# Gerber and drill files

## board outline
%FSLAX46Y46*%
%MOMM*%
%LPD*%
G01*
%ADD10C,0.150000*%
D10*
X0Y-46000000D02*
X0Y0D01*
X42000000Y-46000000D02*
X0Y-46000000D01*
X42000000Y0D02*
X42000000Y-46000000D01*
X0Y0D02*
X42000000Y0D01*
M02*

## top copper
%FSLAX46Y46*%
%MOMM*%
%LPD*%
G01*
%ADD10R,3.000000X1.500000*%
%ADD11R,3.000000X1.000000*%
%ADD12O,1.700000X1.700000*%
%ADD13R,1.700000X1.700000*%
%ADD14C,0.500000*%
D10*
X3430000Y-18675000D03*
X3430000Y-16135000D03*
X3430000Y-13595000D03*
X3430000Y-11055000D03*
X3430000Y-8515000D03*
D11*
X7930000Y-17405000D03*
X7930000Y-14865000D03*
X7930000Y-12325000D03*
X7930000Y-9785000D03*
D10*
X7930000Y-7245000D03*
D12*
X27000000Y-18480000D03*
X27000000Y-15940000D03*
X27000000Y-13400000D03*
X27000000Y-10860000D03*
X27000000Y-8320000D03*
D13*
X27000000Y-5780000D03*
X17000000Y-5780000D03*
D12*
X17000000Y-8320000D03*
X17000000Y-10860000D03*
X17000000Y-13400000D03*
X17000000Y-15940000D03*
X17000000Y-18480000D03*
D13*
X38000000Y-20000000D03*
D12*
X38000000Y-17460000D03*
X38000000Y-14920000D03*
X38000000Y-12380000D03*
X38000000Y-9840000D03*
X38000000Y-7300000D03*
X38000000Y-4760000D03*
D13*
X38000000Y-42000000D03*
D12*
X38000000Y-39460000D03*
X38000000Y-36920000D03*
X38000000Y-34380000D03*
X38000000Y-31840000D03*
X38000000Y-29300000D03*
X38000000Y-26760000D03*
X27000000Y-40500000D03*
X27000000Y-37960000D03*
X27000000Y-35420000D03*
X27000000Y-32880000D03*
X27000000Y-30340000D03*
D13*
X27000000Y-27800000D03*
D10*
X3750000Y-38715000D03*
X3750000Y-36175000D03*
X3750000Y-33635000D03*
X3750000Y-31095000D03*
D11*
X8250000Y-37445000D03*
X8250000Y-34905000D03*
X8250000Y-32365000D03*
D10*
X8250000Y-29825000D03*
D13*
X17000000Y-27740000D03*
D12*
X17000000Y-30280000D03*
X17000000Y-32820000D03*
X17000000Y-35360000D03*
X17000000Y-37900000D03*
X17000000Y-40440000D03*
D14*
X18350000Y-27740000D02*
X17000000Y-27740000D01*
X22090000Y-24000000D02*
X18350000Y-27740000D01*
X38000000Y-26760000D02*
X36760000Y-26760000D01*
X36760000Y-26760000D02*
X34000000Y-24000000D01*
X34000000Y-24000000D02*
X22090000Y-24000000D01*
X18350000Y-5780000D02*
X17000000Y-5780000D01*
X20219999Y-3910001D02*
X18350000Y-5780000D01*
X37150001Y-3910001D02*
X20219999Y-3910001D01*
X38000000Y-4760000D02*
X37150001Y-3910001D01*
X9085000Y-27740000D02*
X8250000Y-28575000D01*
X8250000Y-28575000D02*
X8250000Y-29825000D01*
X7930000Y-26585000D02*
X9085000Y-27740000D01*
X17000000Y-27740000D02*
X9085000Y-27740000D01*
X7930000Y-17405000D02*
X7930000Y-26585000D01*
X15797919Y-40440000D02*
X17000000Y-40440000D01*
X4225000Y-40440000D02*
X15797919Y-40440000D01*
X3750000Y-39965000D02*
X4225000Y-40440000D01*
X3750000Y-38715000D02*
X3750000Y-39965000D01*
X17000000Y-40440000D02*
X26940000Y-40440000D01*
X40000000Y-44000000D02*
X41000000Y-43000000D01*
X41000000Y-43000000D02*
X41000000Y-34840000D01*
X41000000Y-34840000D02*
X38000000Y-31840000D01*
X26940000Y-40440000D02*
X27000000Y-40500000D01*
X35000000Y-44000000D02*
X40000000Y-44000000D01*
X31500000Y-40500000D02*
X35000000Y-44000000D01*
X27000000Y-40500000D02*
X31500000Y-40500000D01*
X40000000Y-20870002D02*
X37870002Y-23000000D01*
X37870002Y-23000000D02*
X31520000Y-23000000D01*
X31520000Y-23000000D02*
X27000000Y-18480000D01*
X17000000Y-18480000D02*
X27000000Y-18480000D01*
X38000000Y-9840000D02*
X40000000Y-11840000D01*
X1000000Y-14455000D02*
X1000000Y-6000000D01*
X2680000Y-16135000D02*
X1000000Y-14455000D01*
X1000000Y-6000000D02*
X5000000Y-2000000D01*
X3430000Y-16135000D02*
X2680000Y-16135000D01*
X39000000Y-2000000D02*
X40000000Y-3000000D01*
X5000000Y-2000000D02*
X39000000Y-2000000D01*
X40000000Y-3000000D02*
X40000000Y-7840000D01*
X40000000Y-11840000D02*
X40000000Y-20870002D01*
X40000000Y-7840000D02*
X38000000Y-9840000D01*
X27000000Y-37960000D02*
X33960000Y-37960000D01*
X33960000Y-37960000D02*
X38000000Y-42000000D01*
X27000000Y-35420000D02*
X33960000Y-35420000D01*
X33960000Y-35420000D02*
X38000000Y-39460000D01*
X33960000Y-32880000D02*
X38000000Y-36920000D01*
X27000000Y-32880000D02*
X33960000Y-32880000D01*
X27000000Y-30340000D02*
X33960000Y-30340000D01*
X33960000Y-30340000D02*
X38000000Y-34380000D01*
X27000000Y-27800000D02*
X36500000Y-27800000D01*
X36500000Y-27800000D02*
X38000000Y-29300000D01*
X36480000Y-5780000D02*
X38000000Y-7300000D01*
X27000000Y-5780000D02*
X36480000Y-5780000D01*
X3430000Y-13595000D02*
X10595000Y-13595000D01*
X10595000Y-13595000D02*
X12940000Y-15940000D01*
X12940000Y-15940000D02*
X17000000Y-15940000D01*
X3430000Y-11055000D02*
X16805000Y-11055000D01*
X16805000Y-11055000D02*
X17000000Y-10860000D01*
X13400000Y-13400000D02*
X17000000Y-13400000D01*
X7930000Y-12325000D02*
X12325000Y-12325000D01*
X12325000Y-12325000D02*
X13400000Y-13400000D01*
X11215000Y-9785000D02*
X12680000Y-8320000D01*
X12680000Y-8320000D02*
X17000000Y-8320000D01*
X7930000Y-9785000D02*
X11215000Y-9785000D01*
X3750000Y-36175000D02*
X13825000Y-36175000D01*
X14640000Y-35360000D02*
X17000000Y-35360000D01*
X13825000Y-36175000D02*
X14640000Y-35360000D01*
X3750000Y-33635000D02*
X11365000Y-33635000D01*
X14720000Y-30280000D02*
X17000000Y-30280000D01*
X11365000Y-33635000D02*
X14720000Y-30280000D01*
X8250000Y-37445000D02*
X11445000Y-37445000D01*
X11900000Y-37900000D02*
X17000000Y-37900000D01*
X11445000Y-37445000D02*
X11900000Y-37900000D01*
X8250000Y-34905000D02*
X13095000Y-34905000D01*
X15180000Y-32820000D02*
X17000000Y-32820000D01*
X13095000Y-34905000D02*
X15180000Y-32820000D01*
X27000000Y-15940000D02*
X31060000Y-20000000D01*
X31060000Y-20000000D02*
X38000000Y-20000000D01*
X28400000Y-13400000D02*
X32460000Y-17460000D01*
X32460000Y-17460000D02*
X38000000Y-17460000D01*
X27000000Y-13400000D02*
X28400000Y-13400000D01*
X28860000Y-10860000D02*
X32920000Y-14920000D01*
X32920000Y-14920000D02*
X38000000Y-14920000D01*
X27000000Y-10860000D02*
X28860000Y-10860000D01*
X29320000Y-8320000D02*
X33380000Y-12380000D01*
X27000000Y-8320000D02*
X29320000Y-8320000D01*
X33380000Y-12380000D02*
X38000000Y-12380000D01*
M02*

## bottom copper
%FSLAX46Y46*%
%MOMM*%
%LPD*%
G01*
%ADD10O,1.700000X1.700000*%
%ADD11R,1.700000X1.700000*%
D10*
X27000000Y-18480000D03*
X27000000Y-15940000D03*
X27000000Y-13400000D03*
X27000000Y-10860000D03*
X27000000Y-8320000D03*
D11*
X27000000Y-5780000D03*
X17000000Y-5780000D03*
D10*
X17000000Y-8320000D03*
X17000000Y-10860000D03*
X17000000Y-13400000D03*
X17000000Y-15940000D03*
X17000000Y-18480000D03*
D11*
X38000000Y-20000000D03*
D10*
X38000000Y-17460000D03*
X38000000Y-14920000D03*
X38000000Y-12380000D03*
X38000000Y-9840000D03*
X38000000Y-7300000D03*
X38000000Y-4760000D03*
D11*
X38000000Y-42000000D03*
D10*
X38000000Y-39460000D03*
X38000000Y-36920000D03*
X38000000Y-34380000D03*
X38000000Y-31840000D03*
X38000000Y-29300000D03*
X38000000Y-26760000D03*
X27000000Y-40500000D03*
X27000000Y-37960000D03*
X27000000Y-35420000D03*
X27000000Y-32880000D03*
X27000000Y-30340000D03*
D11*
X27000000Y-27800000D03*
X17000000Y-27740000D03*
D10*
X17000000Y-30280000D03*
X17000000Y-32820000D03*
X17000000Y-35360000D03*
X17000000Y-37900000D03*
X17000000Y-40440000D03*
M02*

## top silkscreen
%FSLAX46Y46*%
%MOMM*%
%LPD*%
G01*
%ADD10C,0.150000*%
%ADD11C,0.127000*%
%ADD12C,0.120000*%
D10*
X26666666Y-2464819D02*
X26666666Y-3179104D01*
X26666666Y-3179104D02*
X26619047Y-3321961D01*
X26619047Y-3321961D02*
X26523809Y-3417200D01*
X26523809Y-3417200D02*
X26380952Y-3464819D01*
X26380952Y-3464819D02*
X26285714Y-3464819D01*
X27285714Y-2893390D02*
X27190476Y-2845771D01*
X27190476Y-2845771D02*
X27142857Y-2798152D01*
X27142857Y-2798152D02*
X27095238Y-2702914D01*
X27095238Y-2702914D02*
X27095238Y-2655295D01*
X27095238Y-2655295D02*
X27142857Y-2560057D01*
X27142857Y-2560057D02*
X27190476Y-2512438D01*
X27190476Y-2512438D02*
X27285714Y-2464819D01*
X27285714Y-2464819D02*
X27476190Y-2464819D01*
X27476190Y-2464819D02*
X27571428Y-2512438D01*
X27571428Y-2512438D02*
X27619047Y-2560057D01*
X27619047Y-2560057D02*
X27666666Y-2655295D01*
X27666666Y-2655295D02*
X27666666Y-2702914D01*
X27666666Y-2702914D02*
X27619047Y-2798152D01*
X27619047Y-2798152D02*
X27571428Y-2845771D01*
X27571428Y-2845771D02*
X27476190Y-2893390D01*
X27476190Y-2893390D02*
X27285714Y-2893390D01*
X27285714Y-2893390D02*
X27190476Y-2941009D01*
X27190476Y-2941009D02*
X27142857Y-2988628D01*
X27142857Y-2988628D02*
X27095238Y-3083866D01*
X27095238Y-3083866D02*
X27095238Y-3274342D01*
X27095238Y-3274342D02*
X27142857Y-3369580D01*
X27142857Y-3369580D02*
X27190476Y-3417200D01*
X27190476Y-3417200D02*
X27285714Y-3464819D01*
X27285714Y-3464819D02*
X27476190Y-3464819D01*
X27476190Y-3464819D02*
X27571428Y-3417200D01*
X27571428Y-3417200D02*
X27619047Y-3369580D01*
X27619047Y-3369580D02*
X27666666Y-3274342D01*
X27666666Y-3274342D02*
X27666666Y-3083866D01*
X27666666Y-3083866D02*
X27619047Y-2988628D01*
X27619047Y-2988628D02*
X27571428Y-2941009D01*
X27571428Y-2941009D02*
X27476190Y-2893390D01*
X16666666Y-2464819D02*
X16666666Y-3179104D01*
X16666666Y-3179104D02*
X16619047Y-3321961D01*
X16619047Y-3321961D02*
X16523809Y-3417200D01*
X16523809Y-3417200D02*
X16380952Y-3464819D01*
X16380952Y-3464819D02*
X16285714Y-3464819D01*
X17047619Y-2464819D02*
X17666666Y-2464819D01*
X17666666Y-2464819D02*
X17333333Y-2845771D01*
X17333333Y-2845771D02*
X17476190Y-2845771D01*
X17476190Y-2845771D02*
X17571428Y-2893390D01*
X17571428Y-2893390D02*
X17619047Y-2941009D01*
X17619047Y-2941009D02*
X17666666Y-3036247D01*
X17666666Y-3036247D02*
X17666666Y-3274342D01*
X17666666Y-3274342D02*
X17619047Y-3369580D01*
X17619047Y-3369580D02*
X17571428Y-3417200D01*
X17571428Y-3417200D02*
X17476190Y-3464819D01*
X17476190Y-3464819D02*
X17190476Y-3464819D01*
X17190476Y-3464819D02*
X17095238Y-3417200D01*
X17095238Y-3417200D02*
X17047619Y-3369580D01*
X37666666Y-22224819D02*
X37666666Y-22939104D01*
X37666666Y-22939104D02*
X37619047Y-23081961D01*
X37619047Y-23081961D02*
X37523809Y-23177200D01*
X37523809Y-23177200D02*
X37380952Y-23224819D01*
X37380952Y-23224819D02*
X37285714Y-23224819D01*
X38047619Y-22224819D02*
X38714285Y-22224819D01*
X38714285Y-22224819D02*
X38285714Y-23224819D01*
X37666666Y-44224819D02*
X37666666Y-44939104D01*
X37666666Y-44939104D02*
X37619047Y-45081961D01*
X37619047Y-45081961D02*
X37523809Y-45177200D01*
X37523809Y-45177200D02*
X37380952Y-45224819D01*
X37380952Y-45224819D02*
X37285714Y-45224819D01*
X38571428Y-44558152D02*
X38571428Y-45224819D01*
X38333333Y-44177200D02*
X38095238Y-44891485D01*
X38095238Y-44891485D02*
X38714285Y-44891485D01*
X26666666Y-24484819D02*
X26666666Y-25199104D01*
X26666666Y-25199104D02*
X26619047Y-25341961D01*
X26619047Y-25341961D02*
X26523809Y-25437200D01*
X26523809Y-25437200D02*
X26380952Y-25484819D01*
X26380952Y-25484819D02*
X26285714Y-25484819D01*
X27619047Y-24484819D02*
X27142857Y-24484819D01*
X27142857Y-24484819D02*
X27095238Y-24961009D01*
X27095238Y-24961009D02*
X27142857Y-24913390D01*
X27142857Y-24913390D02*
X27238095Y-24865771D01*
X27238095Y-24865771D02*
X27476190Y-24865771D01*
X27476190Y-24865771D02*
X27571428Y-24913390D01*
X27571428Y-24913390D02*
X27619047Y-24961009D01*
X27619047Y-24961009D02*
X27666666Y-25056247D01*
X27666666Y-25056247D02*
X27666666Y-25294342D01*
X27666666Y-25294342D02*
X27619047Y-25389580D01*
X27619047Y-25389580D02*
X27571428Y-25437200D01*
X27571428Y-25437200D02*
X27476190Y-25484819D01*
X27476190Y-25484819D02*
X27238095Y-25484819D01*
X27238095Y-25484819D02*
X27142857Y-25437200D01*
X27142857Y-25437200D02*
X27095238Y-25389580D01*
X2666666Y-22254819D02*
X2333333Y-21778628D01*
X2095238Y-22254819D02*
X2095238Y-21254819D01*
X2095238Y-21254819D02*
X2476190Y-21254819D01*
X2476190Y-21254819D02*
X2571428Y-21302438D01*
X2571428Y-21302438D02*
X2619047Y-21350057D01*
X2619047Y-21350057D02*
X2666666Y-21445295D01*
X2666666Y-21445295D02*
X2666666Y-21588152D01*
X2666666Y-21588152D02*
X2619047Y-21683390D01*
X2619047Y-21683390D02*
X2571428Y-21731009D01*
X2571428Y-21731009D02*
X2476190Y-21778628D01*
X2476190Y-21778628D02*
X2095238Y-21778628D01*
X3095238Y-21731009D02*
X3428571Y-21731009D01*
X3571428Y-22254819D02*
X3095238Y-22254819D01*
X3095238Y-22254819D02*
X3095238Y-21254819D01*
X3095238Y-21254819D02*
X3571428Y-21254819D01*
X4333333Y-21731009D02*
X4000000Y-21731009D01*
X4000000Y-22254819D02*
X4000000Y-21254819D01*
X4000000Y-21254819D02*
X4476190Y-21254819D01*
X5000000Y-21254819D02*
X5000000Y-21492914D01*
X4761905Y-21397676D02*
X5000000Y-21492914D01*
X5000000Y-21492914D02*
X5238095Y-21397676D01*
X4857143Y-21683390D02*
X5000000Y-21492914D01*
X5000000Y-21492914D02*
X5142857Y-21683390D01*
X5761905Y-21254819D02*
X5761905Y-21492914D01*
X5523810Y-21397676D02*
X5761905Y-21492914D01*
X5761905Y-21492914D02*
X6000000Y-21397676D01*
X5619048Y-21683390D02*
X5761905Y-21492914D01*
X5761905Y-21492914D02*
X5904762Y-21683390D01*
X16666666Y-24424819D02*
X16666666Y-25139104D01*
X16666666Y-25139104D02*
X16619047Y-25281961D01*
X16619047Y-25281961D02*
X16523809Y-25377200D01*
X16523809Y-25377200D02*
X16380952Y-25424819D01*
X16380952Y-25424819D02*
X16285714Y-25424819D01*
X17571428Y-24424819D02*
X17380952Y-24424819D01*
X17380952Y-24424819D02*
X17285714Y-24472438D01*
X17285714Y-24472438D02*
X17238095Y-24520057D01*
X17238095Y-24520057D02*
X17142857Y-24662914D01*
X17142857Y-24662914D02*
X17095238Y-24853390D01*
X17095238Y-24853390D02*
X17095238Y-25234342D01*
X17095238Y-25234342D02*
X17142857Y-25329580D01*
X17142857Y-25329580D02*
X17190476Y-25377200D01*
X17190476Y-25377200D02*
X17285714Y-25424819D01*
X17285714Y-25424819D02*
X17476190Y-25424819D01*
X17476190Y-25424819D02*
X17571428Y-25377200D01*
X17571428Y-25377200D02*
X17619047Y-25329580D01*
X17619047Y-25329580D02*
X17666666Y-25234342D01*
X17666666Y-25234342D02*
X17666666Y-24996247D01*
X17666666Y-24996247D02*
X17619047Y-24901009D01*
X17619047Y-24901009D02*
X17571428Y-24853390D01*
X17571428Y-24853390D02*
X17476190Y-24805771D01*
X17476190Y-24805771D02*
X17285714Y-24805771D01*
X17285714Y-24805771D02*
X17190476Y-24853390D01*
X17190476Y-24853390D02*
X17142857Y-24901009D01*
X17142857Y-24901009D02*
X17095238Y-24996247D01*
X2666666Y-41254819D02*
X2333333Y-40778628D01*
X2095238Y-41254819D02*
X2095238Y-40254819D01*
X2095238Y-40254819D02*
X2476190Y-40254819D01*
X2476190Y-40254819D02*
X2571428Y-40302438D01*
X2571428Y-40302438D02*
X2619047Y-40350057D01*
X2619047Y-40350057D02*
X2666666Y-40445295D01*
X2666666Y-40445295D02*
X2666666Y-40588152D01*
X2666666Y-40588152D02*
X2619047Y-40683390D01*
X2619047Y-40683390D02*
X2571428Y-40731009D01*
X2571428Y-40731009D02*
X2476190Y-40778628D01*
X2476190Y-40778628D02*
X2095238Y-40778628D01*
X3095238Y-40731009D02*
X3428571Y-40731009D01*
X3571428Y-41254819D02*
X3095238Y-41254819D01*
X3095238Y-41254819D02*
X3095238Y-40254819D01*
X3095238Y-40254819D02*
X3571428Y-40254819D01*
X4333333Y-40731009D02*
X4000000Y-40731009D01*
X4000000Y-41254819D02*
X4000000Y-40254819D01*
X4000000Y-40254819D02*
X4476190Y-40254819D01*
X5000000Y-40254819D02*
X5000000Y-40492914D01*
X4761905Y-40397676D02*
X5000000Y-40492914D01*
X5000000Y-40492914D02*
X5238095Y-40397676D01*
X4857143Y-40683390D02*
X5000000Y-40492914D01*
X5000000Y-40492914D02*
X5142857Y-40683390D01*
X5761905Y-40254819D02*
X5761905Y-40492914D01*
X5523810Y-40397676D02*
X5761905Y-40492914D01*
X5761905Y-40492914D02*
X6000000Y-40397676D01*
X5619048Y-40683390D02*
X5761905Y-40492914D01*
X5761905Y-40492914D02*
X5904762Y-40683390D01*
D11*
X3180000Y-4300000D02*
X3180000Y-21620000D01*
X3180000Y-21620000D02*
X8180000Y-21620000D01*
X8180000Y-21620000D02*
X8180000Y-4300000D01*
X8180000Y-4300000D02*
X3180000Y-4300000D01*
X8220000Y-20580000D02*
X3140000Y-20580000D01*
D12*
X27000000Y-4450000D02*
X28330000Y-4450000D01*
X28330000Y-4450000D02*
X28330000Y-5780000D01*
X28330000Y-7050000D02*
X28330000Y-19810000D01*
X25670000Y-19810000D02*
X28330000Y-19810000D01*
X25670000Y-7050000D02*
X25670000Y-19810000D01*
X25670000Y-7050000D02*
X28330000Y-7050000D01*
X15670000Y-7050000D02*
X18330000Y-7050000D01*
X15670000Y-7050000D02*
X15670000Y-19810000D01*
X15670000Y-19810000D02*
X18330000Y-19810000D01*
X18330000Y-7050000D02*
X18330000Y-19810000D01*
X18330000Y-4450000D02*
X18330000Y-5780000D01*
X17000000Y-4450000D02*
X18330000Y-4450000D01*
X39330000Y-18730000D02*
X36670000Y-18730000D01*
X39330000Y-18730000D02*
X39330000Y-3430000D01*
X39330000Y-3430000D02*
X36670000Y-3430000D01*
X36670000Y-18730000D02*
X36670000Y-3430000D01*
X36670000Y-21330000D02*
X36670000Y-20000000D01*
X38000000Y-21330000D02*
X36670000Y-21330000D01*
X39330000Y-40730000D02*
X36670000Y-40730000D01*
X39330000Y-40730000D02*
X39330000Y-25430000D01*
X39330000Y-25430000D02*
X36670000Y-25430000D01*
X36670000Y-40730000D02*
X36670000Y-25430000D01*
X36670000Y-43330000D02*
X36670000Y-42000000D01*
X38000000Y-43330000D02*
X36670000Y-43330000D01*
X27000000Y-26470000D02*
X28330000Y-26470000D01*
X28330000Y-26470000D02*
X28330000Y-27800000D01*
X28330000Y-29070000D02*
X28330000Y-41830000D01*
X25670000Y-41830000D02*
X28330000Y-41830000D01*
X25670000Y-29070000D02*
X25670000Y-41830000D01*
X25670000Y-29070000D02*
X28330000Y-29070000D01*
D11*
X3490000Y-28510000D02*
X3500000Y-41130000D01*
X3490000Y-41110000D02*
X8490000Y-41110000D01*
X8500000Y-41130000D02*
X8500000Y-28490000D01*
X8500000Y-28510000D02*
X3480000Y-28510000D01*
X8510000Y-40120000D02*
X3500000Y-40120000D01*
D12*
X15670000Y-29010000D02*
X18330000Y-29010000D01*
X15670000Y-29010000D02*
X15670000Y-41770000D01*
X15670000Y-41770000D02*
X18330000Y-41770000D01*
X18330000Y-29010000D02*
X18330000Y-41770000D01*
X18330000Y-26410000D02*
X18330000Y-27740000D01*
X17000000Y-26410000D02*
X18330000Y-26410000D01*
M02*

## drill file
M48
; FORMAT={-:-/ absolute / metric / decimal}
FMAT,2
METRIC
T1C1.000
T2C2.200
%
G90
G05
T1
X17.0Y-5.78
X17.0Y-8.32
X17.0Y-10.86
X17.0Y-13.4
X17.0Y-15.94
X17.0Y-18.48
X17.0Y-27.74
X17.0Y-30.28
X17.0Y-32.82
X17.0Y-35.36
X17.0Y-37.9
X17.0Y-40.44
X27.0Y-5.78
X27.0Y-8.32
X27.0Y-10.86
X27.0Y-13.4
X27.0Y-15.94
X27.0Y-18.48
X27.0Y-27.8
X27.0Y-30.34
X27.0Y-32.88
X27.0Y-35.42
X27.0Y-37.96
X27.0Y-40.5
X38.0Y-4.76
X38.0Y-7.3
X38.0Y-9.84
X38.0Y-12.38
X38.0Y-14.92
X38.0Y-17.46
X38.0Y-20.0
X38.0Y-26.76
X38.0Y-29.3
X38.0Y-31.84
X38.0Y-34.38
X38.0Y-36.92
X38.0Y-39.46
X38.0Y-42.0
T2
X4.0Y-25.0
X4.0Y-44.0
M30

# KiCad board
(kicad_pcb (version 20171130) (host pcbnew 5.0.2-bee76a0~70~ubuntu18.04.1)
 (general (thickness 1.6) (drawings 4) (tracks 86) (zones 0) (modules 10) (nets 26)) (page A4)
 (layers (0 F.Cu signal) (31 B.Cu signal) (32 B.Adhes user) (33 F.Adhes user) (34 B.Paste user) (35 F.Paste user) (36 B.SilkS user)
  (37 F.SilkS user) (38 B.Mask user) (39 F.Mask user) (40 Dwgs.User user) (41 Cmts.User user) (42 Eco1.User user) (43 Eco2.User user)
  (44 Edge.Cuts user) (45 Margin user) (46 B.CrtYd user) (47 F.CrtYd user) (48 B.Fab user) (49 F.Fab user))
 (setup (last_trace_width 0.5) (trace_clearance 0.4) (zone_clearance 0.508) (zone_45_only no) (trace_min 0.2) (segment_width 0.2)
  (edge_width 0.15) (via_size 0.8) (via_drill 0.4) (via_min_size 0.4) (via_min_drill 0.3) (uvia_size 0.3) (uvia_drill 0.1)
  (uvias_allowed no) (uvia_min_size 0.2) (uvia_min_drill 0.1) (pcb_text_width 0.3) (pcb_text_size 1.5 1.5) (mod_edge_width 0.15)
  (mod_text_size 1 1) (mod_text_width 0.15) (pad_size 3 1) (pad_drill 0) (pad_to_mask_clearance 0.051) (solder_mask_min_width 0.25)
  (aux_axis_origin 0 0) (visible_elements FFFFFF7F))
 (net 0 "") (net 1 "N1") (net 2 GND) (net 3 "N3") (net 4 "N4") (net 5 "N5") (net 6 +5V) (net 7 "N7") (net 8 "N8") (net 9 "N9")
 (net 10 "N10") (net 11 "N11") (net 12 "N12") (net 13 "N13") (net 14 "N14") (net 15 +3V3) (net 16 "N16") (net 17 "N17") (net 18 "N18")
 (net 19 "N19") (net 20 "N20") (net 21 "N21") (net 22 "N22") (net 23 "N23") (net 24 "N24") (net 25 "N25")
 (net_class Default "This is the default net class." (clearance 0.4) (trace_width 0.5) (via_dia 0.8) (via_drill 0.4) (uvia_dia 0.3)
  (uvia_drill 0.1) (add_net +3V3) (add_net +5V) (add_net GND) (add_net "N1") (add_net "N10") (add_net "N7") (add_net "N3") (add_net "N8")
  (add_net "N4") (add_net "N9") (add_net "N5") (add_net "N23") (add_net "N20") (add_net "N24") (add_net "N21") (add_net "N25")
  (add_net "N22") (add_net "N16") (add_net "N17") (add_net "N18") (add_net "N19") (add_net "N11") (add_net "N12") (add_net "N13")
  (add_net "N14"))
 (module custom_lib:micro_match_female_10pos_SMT (layer F.Cu) (at 5.68 12.96 90)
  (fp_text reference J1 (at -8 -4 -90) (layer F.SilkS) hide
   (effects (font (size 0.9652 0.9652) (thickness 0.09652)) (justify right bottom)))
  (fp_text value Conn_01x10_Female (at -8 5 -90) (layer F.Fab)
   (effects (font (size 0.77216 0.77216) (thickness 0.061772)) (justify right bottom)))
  (fp_line (start 8.66 -2.5) (end -8.66 -2.5) (layer F.SilkS) (width 0.127))
  (fp_line (start -8.66 -2.5) (end -8.66 2.5) (layer F.SilkS) (width 0.127))
  (fp_line (start -8.66 2.5) (end 8.66 2.5) (layer F.SilkS) (width 0.127))
  (fp_line (start 8.66 2.5) (end 8.66 -2.5) (layer F.SilkS) (width 0.127))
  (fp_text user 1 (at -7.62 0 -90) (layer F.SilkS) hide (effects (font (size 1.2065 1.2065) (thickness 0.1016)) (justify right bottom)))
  (fp_line (start -7.62 2.54) (end -7.62 -2.54) (layer F.SilkS) (width 0.127))
  (pad 1 smd rect (at -5.715 -2.25 180) (size 3 1.5) (layers F.Cu F.Paste F.Mask) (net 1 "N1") (solder_mask_margin 0.075))
  (pad 3 smd rect (at -3.175 -2.25 180) (size 3 1.5) (layers F.Cu F.Paste F.Mask) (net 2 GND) (solder_mask_margin 0.075))
  (pad 5 smd rect (at -0.635 -2.25 180) (size 3 1.5) (layers F.Cu F.Paste F.Mask) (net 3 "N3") (solder_mask_margin 0.075))
  (pad 7 smd rect (at 1.905 -2.25 180) (size 3 1.5) (layers F.Cu F.Paste F.Mask) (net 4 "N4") (solder_mask_margin 0.075))
  (pad 9 smd rect (at 4.445 -2.25 180) (size 3 1.5) (layers F.Cu F.Paste F.Mask) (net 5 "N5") (solder_mask_margin 0.075))
  (pad 2 smd rect (at -4.445 2.25 180) (size 3 1) (layers F.Cu F.Paste F.Mask) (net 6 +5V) (solder_mask_margin 0.075))
  (pad 4 smd rect (at -1.905 2.25 180) (size 3 1) (layers F.Cu F.Paste F.Mask) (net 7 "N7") (solder_mask_margin 0.075))
  (pad 6 smd rect (at 0.635 2.25 180) (size 3 1) (layers F.Cu F.Paste F.Mask) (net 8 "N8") (solder_mask_margin 0.075))
  (pad 8 smd rect (at 3.175 2.25 180) (size 3 1) (layers F.Cu F.Paste F.Mask) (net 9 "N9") (solder_mask_margin 0.075))
  (pad 10 smd rect (at 5.715 2.25 180) (size 3 1.5) (layers F.Cu F.Paste F.Mask) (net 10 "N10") (solder_mask_margin 0.075)))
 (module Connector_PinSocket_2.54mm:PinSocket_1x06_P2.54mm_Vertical (layer F.Cu) (at 27 5.78)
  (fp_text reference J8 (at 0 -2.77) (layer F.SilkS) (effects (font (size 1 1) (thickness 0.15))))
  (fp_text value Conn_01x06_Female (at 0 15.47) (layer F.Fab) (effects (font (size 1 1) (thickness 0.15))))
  (fp_line (start 0 -1.33) (end 1.33 -1.33) (layer F.SilkS) (width 0.12))
  (fp_line (start 1.33 -1.33) (end 1.33 0) (layer F.SilkS) (width 0.12))
  (fp_line (start 1.33 1.27) (end 1.33 14.03) (layer F.SilkS) (width 0.12))
  (fp_line (start -1.33 14.03) (end 1.33 14.03) (layer F.SilkS) (width 0.12))
  (fp_line (start -1.33 1.27) (end -1.33 14.03) (layer F.SilkS) (width 0.12))
  (fp_line (start -1.33 1.27) (end 1.33 1.27) (layer F.SilkS) (width 0.12))
  (pad 6 thru_hole oval (at 0 12.7) (size 1.7 1.7) (drill 1) (layers *.Cu *.Mask) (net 2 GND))
  (pad 5 thru_hole oval (at 0 10.16) (size 1.7 1.7) (drill 1) (layers *.Cu *.Mask) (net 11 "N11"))
  (pad 4 thru_hole oval (at 0 7.62) (size 1.7 1.7) (drill 1) (layers *.Cu *.Mask) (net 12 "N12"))
  (pad 3 thru_hole oval (at 0 5.08) (size 1.7 1.7) (drill 1) (layers *.Cu *.Mask) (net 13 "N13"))
  (pad 2 thru_hole oval (at 0 2.54) (size 1.7 1.7) (drill 1) (layers *.Cu *.Mask) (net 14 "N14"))
  (pad 1 thru_hole rect (at 0 0) (size 1.7 1.7) (drill 1) (layers *.Cu *.Mask) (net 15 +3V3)))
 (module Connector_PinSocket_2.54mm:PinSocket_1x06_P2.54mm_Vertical (layer F.Cu) (at 17 5.78)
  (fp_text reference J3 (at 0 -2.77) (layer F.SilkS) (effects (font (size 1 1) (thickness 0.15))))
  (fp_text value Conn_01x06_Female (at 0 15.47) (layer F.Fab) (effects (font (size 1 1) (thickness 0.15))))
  (fp_line (start -1.33 1.27) (end 1.33 1.27) (layer F.SilkS) (width 0.12))
  (fp_line (start -1.33 1.27) (end -1.33 14.03) (layer F.SilkS) (width 0.12))
  (fp_line (start -1.33 14.03) (end 1.33 14.03) (layer F.SilkS) (width 0.12))
  (fp_line (start 1.33 1.27) (end 1.33 14.03) (layer F.SilkS) (width 0.12))
  (fp_line (start 1.33 -1.33) (end 1.33 0) (layer F.SilkS) (width 0.12))
  (fp_line (start 0 -1.33) (end 1.33 -1.33) (layer F.SilkS) (width 0.12))
  (pad 1 thru_hole rect (at 0 0) (size 1.7 1.7) (drill 1) (layers *.Cu *.Mask) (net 6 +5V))
  (pad 2 thru_hole oval (at 0 2.54) (size 1.7 1.7) (drill 1) (layers *.Cu *.Mask) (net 9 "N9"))
  (pad 3 thru_hole oval (at 0 5.08) (size 1.7 1.7) (drill 1) (layers *.Cu *.Mask) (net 4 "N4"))
  (pad 4 thru_hole oval (at 0 7.62) (size 1.7 1.7) (drill 1) (layers *.Cu *.Mask) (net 8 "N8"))
  (pad 5 thru_hole oval (at 0 10.16) (size 1.7 1.7) (drill 1) (layers *.Cu *.Mask) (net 3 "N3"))
  (pad 6 thru_hole oval (at 0 12.7) (size 1.7 1.7) (drill 1) (layers *.Cu *.Mask) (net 2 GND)))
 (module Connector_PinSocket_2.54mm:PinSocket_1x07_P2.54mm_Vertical (layer F.Cu) (at 38 20 180)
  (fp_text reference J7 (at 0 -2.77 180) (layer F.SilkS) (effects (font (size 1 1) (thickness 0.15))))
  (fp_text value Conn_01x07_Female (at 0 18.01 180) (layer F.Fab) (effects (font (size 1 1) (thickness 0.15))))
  (fp_line (start -1.33 1.27) (end 1.33 1.27) (layer F.SilkS) (width 0.12))
  (fp_line (start -1.33 1.27) (end -1.33 16.57) (layer F.SilkS) (width 0.12))
  (fp_line (start -1.33 16.57) (end 1.33 16.57) (layer F.SilkS) (width 0.12))
  (fp_line (start 1.33 1.27) (end 1.33 16.57) (layer F.SilkS) (width 0.12))
  (fp_line (start 1.33 -1.33) (end 1.33 0) (layer F.SilkS) (width 0.12))
  (fp_line (start 0 -1.33) (end 1.33 -1.33) (layer F.SilkS) (width 0.12))
  (pad 1 thru_hole rect (at 0 0 180) (size 1.7 1.7) (drill 1) (layers *.Cu *.Mask) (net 11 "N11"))
  (pad 2 thru_hole oval (at 0 2.54 180) (size 1.7 1.7) (drill 1) (layers *.Cu *.Mask) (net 12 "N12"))
  (pad 3 thru_hole oval (at 0 5.08 180) (size 1.7 1.7) (drill 1) (layers *.Cu *.Mask) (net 13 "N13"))
  (pad 4 thru_hole oval (at 0 7.62 180) (size 1.7 1.7) (drill 1) (layers *.Cu *.Mask) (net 14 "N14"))
  (pad 5 thru_hole oval (at 0 10.16 180) (size 1.7 1.7) (drill 1) (layers *.Cu *.Mask) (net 2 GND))
  (pad 6 thru_hole oval (at 0 12.7 180) (size 1.7 1.7) (drill 1) (layers *.Cu *.Mask) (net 15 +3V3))
  (pad 7 thru_hole oval (at 0 15.24 180) (size 1.7 1.7) (drill 1) (layers *.Cu *.Mask) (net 6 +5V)))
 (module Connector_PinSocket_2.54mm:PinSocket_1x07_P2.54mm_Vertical (layer F.Cu) (at 38 42 180)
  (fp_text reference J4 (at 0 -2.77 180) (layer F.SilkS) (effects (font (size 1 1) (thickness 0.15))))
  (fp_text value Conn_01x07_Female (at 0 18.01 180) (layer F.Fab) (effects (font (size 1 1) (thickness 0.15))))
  (fp_line (start -1.33 1.27) (end 1.33 1.27) (layer F.SilkS) (width 0.12))
  (fp_line (start -1.33 1.27) (end -1.33 16.57) (layer F.SilkS) (width 0.12))
  (fp_line (start -1.33 16.57) (end 1.33 16.57) (layer F.SilkS) (width 0.12))
  (fp_line (start 1.33 1.27) (end 1.33 16.57) (layer F.SilkS) (width 0.12))
  (fp_line (start 1.33 -1.33) (end 1.33 0) (layer F.SilkS) (width 0.12))
  (fp_line (start 0 -1.33) (end 1.33 -1.33) (layer F.SilkS) (width 0.12))
  (pad 1 thru_hole rect (at 0 0 180) (size 1.7 1.7) (drill 1) (layers *.Cu *.Mask) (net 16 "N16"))
  (pad 2 thru_hole oval (at 0 2.54 180) (size 1.7 1.7) (drill 1) (layers *.Cu *.Mask) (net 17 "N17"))
  (pad 3 thru_hole oval (at 0 5.08 180) (size 1.7 1.7) (drill 1) (layers *.Cu *.Mask) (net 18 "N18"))
  (pad 4 thru_hole oval (at 0 7.62 180) (size 1.7 1.7) (drill 1) (layers *.Cu *.Mask) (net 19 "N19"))
  (pad 5 thru_hole oval (at 0 10.16 180) (size 1.7 1.7) (drill 1) (layers *.Cu *.Mask) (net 2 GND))
  (pad 6 thru_hole oval (at 0 12.7 180) (size 1.7 1.7) (drill 1) (layers *.Cu *.Mask) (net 15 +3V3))
  (pad 7 thru_hole oval (at 0 15.24 180) (size 1.7 1.7) (drill 1) (layers *.Cu *.Mask) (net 6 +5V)))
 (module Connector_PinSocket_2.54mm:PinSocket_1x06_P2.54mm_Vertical (layer F.Cu) (at 27 27.8)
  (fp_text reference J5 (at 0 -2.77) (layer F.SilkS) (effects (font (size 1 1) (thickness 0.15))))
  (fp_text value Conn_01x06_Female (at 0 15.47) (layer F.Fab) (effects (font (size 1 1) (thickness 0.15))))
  (fp_line (start 0 -1.33) (end 1.33 -1.33) (layer F.SilkS) (width 0.12))
  (fp_line (start 1.33 -1.33) (end 1.33 0) (layer F.SilkS) (width 0.12))
  (fp_line (start 1.33 1.27) (end 1.33 14.03) (layer F.SilkS) (width 0.12))
  (fp_line (start -1.33 14.03) (end 1.33 14.03) (layer F.SilkS) (width 0.12))
  (fp_line (start -1.33 1.27) (end -1.33 14.03) (layer F.SilkS) (width 0.12))
  (fp_line (start -1.33 1.27) (end 1.33 1.27) (layer F.SilkS) (width 0.12))
  (pad 6 thru_hole oval (at 0 12.7) (size 1.7 1.7) (drill 1) (layers *.Cu *.Mask) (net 2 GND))
  (pad 5 thru_hole oval (at 0 10.16) (size 1.7 1.7) (drill 1) (layers *.Cu *.Mask) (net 16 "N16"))
  (pad 4 thru_hole oval (at 0 7.62) (size 1.7 1.7) (drill 1) (layers *.Cu *.Mask) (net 17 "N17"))
  (pad 3 thru_hole oval (at 0 5.08) (size 1.7 1.7) (drill 1) (layers *.Cu *.Mask) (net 18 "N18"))
  (pad 2 thru_hole oval (at 0 2.54) (size 1.7 1.7) (drill 1) (layers *.Cu *.Mask) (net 19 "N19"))
  (pad 1 thru_hole rect (at 0 0) (size 1.7 1.7) (drill 1) (layers *.Cu *.Mask) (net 15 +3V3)))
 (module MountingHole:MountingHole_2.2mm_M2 (layer F.Cu) (at 4 25)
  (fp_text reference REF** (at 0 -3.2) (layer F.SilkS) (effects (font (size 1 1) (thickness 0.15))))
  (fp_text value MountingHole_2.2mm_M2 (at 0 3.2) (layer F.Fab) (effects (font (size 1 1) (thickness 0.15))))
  (pad 1 np_thru_hole circle (at 0 0) (size 2.2 2.2) (drill 2.2) (layers *.Cu *.Mask)))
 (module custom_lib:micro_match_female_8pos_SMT (layer F.Cu) (at 6 33 90)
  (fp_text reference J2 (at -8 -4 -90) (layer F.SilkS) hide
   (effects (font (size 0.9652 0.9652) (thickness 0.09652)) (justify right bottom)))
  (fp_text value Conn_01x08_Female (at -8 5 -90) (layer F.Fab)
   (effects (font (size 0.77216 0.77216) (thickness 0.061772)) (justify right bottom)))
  (fp_line (start 4.49 -2.51) (end -8.13 -2.5) (layer F.SilkS) (width 0.127))
  (fp_line (start -8.11 -2.51) (end -8.11 2.49) (layer F.SilkS) (width 0.127))
  (fp_line (start -8.13 2.5) (end 4.51 2.5) (layer F.SilkS) (width 0.127))
  (fp_line (start 4.49 2.5) (end 4.49 -2.52) (layer F.SilkS) (width 0.127))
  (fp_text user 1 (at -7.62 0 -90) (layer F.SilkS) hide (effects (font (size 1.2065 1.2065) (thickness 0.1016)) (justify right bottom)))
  (fp_line (start -7.12 2.51) (end -7.12 -2.5) (layer F.SilkS) (width 0.127))
  (pad 1 smd rect (at -5.715 -2.25 180) (size 3 1.5) (layers F.Cu F.Paste F.Mask) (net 2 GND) (solder_mask_margin 0.075))
  (pad 3 smd rect (at -3.175 -2.25 180) (size 3 1.5) (layers F.Cu F.Paste F.Mask) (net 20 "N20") (solder_mask_margin 0.075))
  (pad 5 smd rect (at -0.635 -2.25 180) (size 3 1.5) (layers F.Cu F.Paste F.Mask) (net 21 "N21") (solder_mask_margin 0.075))
  (pad 7 smd rect (at 1.905 -2.25 180) (size 3 1.5) (layers F.Cu F.Paste F.Mask) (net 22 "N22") (solder_mask_margin 0.075))
  (pad 2 smd rect (at -4.445 2.25 180) (size 3 1) (layers F.Cu F.Paste F.Mask) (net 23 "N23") (solder_mask_margin 0.075))
  (pad 4 smd rect (at -1.905 2.25 180) (size 3 1) (layers F.Cu F.Paste F.Mask) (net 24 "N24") (solder_mask_margin 0.075))
  (pad 6 smd rect (at 0.635 2.25 180) (size 3 1) (layers F.Cu F.Paste F.Mask) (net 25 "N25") (solder_mask_margin 0.075))
  (pad 8 smd rect (at 3.175 2.25 180) (size 3 1.5) (layers F.Cu F.Paste F.Mask) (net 6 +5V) (solder_mask_margin 0.075)))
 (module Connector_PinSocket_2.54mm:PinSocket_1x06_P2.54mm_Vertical (layer F.Cu) (at 17 27.74)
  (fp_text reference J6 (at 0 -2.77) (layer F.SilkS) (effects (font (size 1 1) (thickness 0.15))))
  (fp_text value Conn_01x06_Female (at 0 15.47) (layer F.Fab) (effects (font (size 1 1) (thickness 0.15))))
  (fp_line (start -1.33 1.27) (end 1.33 1.27) (layer F.SilkS) (width 0.12))
  (fp_line (start -1.33 1.27) (end -1.33 14.03) (layer F.SilkS) (width 0.12))
  (fp_line (start -1.33 14.03) (end 1.33 14.03) (layer F.SilkS) (width 0.12))
  (fp_line (start 1.33 1.27) (end 1.33 14.03) (layer F.SilkS) (width 0.12))
  (fp_line (start 1.33 -1.33) (end 1.33 0) (layer F.SilkS) (width 0.12))
  (fp_line (start 0 -1.33) (end 1.33 -1.33) (layer F.SilkS) (width 0.12))
  (pad 1 thru_hole rect (at 0 0) (size 1.7 1.7) (drill 1) (layers *.Cu *.Mask) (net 6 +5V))
  (pad 2 thru_hole oval (at 0 2.54) (size 1.7 1.7) (drill 1) (layers *.Cu *.Mask) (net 21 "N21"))
  (pad 3 thru_hole oval (at 0 5.08) (size 1.7 1.7) (drill 1) (layers *.Cu *.Mask) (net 24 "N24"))
  (pad 4 thru_hole oval (at 0 7.62) (size 1.7 1.7) (drill 1) (layers *.Cu *.Mask) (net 20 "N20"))
  (pad 5 thru_hole oval (at 0 10.16) (size 1.7 1.7) (drill 1) (layers *.Cu *.Mask) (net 23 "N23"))
  (pad 6 thru_hole oval (at 0 12.7) (size 1.7 1.7) (drill 1) (layers *.Cu *.Mask) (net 2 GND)))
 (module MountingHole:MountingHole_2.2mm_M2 (layer F.Cu) (at 4 44)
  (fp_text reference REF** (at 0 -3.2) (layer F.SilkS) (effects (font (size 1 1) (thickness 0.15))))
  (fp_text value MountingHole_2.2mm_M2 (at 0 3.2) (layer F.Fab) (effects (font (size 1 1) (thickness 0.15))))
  (pad 1 np_thru_hole circle (at 0 0) (size 2.2 2.2) (drill 2.2) (layers *.Cu *.Mask)))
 (gr_line (start 0 46) (end 0 0) (layer Edge.Cuts) (width 0.15))
 (gr_line (start 42 46) (end 0 46) (layer Edge.Cuts) (width 0.15))
 (gr_line (start 42 0) (end 42 46) (layer Edge.Cuts) (width 0.15))
 (gr_line (start 0 0) (end 42 0) (layer Edge.Cuts) (width 0.15))
 (segment (start 18.35 27.74) (end 17 27.74) (width 0.5) (layer F.Cu) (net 6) (status 1000000))
 (segment (start 22.09 24) (end 18.35 27.74) (width 0.5) (layer F.Cu) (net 6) (status 1000000))
 (segment (start 38 26.76) (end 36.76 26.76) (width 0.5) (layer F.Cu) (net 6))
 (segment (start 36.76 26.76) (end 34 24) (width 0.5) (layer F.Cu) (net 6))
 (segment (start 34 24) (end 22.09 24) (width 0.5) (layer F.Cu) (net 6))
 (segment (start 18.35 5.78) (end 17 5.78) (width 0.5) (layer F.Cu) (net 6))
 (segment (start 20.219999 3.910001) (end 18.35 5.78) (width 0.5) (layer F.Cu) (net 6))
 (segment (start 37.150001 3.910001) (end 20.219999 3.910001) (width 0.5) (layer F.Cu) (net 6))
 (segment (start 38 4.76) (end 37.150001 3.910001) (width 0.5) (layer F.Cu) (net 6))
 (segment (start 9.085 27.74) (end 8.25 28.575) (width 0.5) (layer F.Cu) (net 6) (status 1000000))
 (segment (start 8.25 28.575) (end 8.25 29.825) (width 0.5) (layer F.Cu) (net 6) (status 1000000))
 (segment (start 7.93 26.585) (end 9.085 27.74) (width 0.5) (layer F.Cu) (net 6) (status 1000000))
 (segment (start 17 27.74) (end 9.085 27.74) (width 0.5) (layer F.Cu) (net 6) (status 1000000))
 (segment (start 7.93 17.405) (end 7.93 26.585) (width 0.5) (layer F.Cu) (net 6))
 (segment (start 15.797919 40.44) (end 17 40.44) (width 0.5) (layer F.Cu) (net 2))
 (segment (start 4.225 40.44) (end 15.797919 40.44) (width 0.5) (layer F.Cu) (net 2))
 (segment (start 3.75 39.965) (end 4.225 40.44) (width 0.5) (layer F.Cu) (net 2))
 (segment (start 3.75 38.715) (end 3.75 39.965) (width 0.5) (layer F.Cu) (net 2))
 (segment (start 17 40.44) (end 26.94 40.44) (width 0.5) (layer F.Cu) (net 2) (status 1000000))
 (segment (start 40 44) (end 41 43) (width 0.5) (layer F.Cu) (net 2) (status 1000000))
 (segment (start 41 43) (end 41 34.84) (width 0.5) (layer F.Cu) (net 2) (status 1000000))
 (segment (start 41 34.84) (end 38 31.84) (width 0.5) (layer F.Cu) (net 2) (status 1000000))
 (segment (start 26.94 40.44) (end 27 40.5) (width 0.5) (layer F.Cu) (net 2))
 (segment (start 35 44) (end 40 44) (width 0.5) (layer F.Cu) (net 2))
 (segment (start 31.5 40.5) (end 35 44) (width 0.5) (layer F.Cu) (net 2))
 (segment (start 27 40.5) (end 31.5 40.5) (width 0.5) (layer F.Cu) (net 2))
 (segment (start 40 20.870002) (end 37.870002 23) (width 0.5) (layer F.Cu) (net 2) (status 1000000))
 (segment (start 37.870002 23) (end 31.52 23) (width 0.5) (layer F.Cu) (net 2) (status 1000000))
 (segment (start 31.52 23) (end 27 18.48) (width 0.5) (layer F.Cu) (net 2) (status 1000000))
 (segment (start 17 18.48) (end 27 18.48) (width 0.5) (layer F.Cu) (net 2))
 (segment (start 38 9.84) (end 40 11.84) (width 0.5) (layer F.Cu) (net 2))
 (segment (start 1 14.455) (end 1 6) (width 0.5) (layer F.Cu) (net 2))
 (segment (start 2.68 16.135) (end 1 14.455) (width 0.5) (layer F.Cu) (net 2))
 (segment (start 1 6) (end 5 2) (width 0.5) (layer F.Cu) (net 2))
 (segment (start 3.43 16.135) (end 2.68 16.135) (width 0.5) (layer F.Cu) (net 2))
 (segment (start 39 2) (end 40 3) (width 0.5) (layer F.Cu) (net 2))
 (segment (start 5 2) (end 39 2) (width 0.5) (layer F.Cu) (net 2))
 (segment (start 40 3) (end 40 7.84) (width 0.5) (layer F.Cu) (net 2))
 (segment (start 40 11.84) (end 40 20.870002) (width 0.5) (layer F.Cu) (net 2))
 (segment (start 40 7.84) (end 38 9.84) (width 0.5) (layer F.Cu) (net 2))
 (segment (start 27 37.96) (end 33.96 37.96) (width 0.5) (layer F.Cu) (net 16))
 (segment (start 33.96 37.96) (end 38 42) (width 0.5) (layer F.Cu) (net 16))
 (segment (start 27 35.42) (end 33.96 35.42) (width 0.5) (layer F.Cu) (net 17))
 (segment (start 33.96 35.42) (end 38 39.46) (width 0.5) (layer F.Cu) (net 17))
 (segment (start 33.96 32.88) (end 38 36.92) (width 0.5) (layer F.Cu) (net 18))
 (segment (start 27 32.88) (end 33.96 32.88) (width 0.5) (layer F.Cu) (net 18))
 (segment (start 27 30.34) (end 33.96 30.34) (width 0.5) (layer F.Cu) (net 19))
 (segment (start 33.96 30.34) (end 38 34.38) (width 0.5) (layer F.Cu) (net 19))
 (segment (start 27 27.8) (end 36.5 27.8) (width 0.5) (layer F.Cu) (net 15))
 (segment (start 36.5 27.8) (end 38 29.3) (width 0.5) (layer F.Cu) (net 15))
 (segment (start 36.48 5.78) (end 38 7.3) (width 0.5) (layer F.Cu) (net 15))
 (segment (start 27 5.78) (end 36.48 5.78) (width 0.5) (layer F.Cu) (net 15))
 (segment (start 3.43 13.595) (end 10.595 13.595) (width 0.5) (layer F.Cu) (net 3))
 (segment (start 10.595 13.595) (end 12.94 15.94) (width 0.5) (layer F.Cu) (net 3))
 (segment (start 12.94 15.94) (end 17 15.94) (width 0.5) (layer F.Cu) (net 3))
 (segment (start 3.43 11.055) (end 16.805 11.055) (width 0.5) (layer F.Cu) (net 4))
 (segment (start 16.805 11.055) (end 17 10.86) (width 0.5) (layer F.Cu) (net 4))
 (segment (start 13.4 13.4) (end 17 13.4) (width 0.5) (layer F.Cu) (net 8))
 (segment (start 7.93 12.325) (end 12.325 12.325) (width 0.5) (layer F.Cu) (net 8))
 (segment (start 12.325 12.325) (end 13.4 13.4) (width 0.5) (layer F.Cu) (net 8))
 (segment (start 11.215 9.785) (end 12.68 8.32) (width 0.5) (layer F.Cu) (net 9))
 (segment (start 12.68 8.32) (end 17 8.32) (width 0.5) (layer F.Cu) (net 9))
 (segment (start 7.93 9.785) (end 11.215 9.785) (width 0.5) (layer F.Cu) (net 9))
 (segment (start 3.75 36.175) (end 13.825 36.175) (width 0.5) (layer F.Cu) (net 20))
 (segment (start 14.64 35.36) (end 17 35.36) (width 0.5) (layer F.Cu) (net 20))
 (segment (start 13.825 36.175) (end 14.64 35.36) (width 0.5) (layer F.Cu) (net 20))
 (segment (start 3.75 33.635) (end 11.365 33.635) (width 0.5) (layer F.Cu) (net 21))
 (segment (start 14.72 30.28) (end 17 30.28) (width 0.5) (layer F.Cu) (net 21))
 (segment (start 11.365 33.635) (end 14.72 30.28) (width 0.5) (layer F.Cu) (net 21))
 (segment (start 8.25 37.445) (end 11.445 37.445) (width 0.5) (layer F.Cu) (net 23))
 (segment (start 11.9 37.9) (end 17 37.9) (width 0.5) (layer F.Cu) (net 23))
 (segment (start 11.445 37.445) (end 11.9 37.9) (width 0.5) (layer F.Cu) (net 23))
 (segment (start 8.25 34.905) (end 13.095 34.905) (width 0.5) (layer F.Cu) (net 24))
 (segment (start 15.18 32.82) (end 17 32.82) (width 0.5) (layer F.Cu) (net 24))
 (segment (start 13.095 34.905) (end 15.18 32.82) (width 0.5) (layer F.Cu) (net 24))
 (segment (start 27 15.94) (end 31.06 20) (width 0.5) (layer F.Cu) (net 11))
 (segment (start 31.06 20) (end 38 20) (width 0.5) (layer F.Cu) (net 11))
 (segment (start 28.4 13.4) (end 32.46 17.46) (width 0.5) (layer F.Cu) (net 12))
 (segment (start 32.46 17.46) (end 38 17.46) (width 0.5) (layer F.Cu) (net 12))
 (segment (start 27 13.4) (end 28.4 13.4) (width 0.5) (layer F.Cu) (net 12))
 (segment (start 28.86 10.86) (end 32.92 14.92) (width 0.5) (layer F.Cu) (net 13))
 (segment (start 32.92 14.92) (end 38 14.92) (width 0.5) (layer F.Cu) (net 13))
 (segment (start 27 10.86) (end 28.86 10.86) (width 0.5) (layer F.Cu) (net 13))
 (segment (start 29.32 8.32) (end 33.38 12.38) (width 0.5) (layer F.Cu) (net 14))
 (segment (start 27 8.32) (end 29.32 8.32) (width 0.5) (layer F.Cu) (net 14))
 (segment (start 33.38 12.38) (end 38 12.38) (width 0.5) (layer F.Cu) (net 14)))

